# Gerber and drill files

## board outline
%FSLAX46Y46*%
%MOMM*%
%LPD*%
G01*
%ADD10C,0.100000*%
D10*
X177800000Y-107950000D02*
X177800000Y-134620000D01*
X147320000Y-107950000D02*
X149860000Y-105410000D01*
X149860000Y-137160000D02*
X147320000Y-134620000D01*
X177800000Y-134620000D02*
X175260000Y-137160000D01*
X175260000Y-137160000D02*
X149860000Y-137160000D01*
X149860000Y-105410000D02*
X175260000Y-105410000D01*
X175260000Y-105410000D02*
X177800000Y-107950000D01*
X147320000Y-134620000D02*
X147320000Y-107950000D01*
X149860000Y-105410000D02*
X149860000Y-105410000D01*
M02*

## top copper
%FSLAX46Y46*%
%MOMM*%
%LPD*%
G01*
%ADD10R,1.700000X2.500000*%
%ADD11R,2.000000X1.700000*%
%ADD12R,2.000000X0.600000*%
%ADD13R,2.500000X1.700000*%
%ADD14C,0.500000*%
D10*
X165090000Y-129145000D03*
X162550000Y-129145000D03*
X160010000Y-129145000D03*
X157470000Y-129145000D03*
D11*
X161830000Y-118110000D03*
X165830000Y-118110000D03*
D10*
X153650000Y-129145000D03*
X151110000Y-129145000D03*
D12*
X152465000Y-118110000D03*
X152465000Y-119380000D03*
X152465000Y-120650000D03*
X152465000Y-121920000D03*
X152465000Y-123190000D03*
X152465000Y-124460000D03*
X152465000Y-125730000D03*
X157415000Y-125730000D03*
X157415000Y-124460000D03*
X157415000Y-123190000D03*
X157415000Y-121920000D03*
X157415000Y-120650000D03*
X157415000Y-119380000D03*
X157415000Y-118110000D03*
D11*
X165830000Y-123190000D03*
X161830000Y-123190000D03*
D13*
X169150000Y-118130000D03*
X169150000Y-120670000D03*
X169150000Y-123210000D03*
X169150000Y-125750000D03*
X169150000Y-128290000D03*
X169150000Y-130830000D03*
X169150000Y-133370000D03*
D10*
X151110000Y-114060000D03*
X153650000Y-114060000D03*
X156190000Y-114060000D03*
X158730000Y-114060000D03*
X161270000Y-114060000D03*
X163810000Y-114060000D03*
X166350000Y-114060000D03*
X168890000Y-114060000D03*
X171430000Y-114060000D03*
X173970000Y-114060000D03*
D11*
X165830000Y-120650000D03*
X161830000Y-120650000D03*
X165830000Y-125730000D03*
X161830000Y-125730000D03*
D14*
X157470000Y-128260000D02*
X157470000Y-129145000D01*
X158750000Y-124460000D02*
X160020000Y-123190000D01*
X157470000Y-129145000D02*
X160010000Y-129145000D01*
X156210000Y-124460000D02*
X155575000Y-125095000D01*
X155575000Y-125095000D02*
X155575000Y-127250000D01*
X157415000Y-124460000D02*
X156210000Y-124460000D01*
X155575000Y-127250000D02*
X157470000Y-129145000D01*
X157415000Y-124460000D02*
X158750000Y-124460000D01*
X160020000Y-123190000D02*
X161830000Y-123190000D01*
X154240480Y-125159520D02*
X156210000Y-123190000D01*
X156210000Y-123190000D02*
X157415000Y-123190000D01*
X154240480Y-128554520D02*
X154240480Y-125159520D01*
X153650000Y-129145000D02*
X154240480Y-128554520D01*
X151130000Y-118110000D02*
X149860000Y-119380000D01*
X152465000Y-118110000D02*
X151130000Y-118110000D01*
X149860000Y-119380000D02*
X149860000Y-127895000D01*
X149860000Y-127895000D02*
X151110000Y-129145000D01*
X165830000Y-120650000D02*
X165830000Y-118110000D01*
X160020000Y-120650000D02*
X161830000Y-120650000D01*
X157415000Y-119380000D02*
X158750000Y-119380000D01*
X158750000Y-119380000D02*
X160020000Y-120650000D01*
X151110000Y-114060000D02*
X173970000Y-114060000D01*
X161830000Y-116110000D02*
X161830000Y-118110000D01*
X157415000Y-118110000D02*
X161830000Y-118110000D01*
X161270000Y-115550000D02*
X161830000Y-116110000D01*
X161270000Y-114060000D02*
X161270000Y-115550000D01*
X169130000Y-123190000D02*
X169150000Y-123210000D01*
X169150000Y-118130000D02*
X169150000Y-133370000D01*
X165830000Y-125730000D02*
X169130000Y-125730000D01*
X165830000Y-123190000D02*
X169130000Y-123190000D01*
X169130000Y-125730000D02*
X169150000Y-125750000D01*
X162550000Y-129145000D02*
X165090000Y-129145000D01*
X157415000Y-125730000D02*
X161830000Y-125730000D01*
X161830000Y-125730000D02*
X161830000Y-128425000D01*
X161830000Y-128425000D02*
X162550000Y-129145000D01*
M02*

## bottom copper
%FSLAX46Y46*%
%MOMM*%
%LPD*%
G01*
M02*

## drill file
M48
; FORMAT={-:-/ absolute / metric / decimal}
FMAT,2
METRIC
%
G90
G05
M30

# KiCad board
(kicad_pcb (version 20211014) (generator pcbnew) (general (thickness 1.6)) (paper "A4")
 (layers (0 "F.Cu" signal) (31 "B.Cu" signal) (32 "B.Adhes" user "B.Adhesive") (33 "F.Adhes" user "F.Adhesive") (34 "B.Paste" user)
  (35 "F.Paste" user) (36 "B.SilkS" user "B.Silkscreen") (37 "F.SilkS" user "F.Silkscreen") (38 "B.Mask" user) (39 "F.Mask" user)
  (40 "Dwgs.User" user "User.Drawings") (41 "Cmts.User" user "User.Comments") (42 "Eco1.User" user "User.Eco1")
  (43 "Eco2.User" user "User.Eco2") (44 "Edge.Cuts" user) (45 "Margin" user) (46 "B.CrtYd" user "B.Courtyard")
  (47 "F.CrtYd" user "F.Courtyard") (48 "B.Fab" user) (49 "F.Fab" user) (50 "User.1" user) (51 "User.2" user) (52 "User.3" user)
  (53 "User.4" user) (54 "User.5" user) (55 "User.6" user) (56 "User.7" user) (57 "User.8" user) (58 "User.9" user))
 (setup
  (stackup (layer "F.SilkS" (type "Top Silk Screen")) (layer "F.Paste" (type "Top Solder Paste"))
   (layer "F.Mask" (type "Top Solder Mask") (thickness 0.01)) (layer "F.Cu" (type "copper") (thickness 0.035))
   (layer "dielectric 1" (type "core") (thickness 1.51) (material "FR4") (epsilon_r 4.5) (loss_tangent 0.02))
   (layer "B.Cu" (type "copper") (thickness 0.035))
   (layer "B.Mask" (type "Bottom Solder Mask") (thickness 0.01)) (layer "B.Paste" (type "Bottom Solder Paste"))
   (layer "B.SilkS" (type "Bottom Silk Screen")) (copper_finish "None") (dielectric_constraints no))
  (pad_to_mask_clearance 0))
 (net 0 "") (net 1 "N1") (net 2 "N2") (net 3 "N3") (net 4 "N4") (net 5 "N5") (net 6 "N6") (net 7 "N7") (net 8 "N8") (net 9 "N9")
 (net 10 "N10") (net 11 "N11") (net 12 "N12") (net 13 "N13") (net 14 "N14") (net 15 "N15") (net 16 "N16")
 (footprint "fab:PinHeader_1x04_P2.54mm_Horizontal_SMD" (layer "F.Cu") (at 165.09 129.145 -90)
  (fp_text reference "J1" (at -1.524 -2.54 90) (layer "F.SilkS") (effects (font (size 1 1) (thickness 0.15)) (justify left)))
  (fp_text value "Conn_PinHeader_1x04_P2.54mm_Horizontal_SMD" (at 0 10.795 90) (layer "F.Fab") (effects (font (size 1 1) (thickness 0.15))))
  (pad "1" smd rect locked (at 0 0 270) (size 2.5 1.7) (layers "F.Cu" "F.Paste" "F.Mask") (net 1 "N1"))
  (pad "2" smd rect locked (at 0 2.54 270) (size 2.5 1.7) (layers "F.Cu" "F.Paste" "F.Mask") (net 1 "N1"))
  (pad "3" smd rect locked (at 0 5.08 270) (size 2.5 1.7) (layers "F.Cu" "F.Paste" "F.Mask") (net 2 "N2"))
  (pad "4" smd rect locked (at 0 7.62 270) (size 2.5 1.7) (layers "F.Cu" "F.Paste" "F.Mask") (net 2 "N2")))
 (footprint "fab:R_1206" (layer "F.Cu") (at 163.83 118.11)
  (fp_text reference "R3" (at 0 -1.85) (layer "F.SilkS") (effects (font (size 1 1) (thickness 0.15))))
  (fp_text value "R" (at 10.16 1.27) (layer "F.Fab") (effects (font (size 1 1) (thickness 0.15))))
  (pad "1" smd rect locked (at -2 0) (size 2 1.7) (layers "F.Cu" "F.Paste" "F.Mask") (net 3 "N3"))
  (pad "2" smd rect locked (at 2 0) (size 2 1.7) (layers "F.Cu" "F.Paste" "F.Mask") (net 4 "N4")))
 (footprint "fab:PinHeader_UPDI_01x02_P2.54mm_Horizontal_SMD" (layer "F.Cu") (at 153.65 129.145 -90)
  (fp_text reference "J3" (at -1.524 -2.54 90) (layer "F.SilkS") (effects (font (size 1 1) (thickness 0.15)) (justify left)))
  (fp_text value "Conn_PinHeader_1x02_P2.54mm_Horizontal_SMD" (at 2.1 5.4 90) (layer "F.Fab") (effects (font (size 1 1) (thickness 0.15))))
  (pad "1" smd rect locked (at 0 0 270) (size 2.5 1.7) (layers "F.Cu" "F.Paste" "F.Mask") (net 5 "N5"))
  (pad "2" smd rect locked (at 0 2.54 270) (size 2.5 1.7) (layers "F.Cu" "F.Paste" "F.Mask") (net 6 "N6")))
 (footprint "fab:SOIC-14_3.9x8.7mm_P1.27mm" (layer "F.Cu") (at 154.94 121.92)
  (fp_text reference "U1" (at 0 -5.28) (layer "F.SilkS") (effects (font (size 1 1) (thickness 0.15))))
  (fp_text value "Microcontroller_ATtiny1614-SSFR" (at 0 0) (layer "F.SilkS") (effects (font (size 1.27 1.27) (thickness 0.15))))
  (pad "1" smd rect (at -2.475 -3.81) (size 2 0.6) (layers "F.Cu" "F.Paste" "F.Mask") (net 6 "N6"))
  (pad "2" smd rect (at -2.475 -2.54) (size 2 0.6) (layers "F.Cu" "F.Paste" "F.Mask") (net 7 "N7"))
  (pad "3" smd rect (at -2.475 -1.27) (size 2 0.6) (layers "F.Cu" "F.Paste" "F.Mask") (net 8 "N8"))
  (pad "4" smd rect (at -2.475 0) (size 2 0.6) (layers "F.Cu" "F.Paste" "F.Mask") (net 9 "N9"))
  (pad "5" smd rect (at -2.475 1.27) (size 2 0.6) (layers "F.Cu" "F.Paste" "F.Mask") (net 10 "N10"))
  (pad "6" smd rect (at -2.475 2.54) (size 2 0.6) (layers "F.Cu" "F.Paste" "F.Mask") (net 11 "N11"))
  (pad "7" smd rect (at -2.475 3.81) (size 2 0.6) (layers "F.Cu" "F.Paste" "F.Mask") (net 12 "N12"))
  (pad "8" smd rect (at 2.475 3.81) (size 2 0.6) (layers "F.Cu" "F.Paste" "F.Mask") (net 1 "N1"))
  (pad "9" smd rect (at 2.475 2.54) (size 2 0.6) (layers "F.Cu" "F.Paste" "F.Mask") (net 2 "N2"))
  (pad "10" smd rect (at 2.475 1.27) (size 2 0.6) (layers "F.Cu" "F.Paste" "F.Mask") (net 5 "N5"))
  (pad "11" smd rect (at 2.475 0) (size 2 0.6) (layers "F.Cu" "F.Paste" "F.Mask") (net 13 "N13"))
  (pad "12" smd rect (at 2.475 -1.27) (size 2 0.6) (layers "F.Cu" "F.Paste" "F.Mask") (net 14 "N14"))
  (pad "13" smd rect (at 2.475 -2.54) (size 2 0.6) (layers "F.Cu" "F.Paste" "F.Mask") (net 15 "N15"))
  (pad "14" smd rect (at 2.475 -3.81) (size 2 0.6) (layers "F.Cu" "F.Paste" "F.Mask") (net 3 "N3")))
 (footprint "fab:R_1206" (layer "F.Cu") (at 163.83 123.19 180)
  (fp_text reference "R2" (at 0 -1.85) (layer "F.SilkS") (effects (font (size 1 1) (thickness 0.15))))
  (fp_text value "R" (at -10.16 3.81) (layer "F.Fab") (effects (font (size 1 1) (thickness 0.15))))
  (pad "1" smd rect locked (at -2 0 180) (size 2 1.7) (layers "F.Cu" "F.Paste" "F.Mask") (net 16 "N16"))
  (pad "2" smd rect locked (at 2 0 180) (size 2 1.7) (layers "F.Cu" "F.Paste" "F.Mask") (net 2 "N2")))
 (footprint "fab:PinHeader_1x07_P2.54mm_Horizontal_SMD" (layer "F.Cu") (at 169.15 118.13)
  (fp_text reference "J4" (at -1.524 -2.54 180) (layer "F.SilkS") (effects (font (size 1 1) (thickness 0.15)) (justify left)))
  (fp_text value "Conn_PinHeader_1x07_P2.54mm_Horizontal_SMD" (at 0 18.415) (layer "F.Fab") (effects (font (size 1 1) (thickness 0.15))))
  (pad "1" smd rect locked (at 0 0) (size 2.5 1.7) (layers "F.Cu" "F.Paste" "F.Mask") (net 16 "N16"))
  (pad "2" smd rect locked (at 0 2.54) (size 2.5 1.7) (layers "F.Cu" "F.Paste" "F.Mask") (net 16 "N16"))
  (pad "3" smd rect locked (at 0 5.08) (size 2.5 1.7) (layers "F.Cu" "F.Paste" "F.Mask") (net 16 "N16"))
  (pad "4" smd rect locked (at 0 7.62) (size 2.5 1.7) (layers "F.Cu" "F.Paste" "F.Mask") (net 16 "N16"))
  (pad "5" smd rect locked (at 0 10.16) (size 2.5 1.7) (layers "F.Cu" "F.Paste" "F.Mask") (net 16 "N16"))
  (pad "6" smd rect locked (at 0 12.7) (size 2.5 1.7) (layers "F.Cu" "F.Paste" "F.Mask") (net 16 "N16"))
  (pad "7" smd rect locked (at 0 15.24) (size 2.5 1.7) (layers "F.Cu" "F.Paste" "F.Mask") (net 16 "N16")))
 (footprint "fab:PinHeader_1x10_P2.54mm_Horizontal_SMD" (layer "F.Cu") (at 151.11 114.06 90)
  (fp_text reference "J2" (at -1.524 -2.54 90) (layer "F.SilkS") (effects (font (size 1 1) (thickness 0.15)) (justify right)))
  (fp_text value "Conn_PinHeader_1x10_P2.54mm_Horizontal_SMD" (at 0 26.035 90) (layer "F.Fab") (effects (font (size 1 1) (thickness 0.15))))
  (pad "1" smd rect locked (at 0 0 90) (size 2.5 1.7) (layers "F.Cu" "F.Paste" "F.Mask") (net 3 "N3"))
  (pad "2" smd rect locked (at 0 2.54 90) (size 2.5 1.7) (layers "F.Cu" "F.Paste" "F.Mask") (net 3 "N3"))
  (pad "3" smd rect locked (at 0 5.08 90) (size 2.5 1.7) (layers "F.Cu" "F.Paste" "F.Mask") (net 3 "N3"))
  (pad "4" smd rect locked (at 0 7.62 90) (size 2.5 1.7) (layers "F.Cu" "F.Paste" "F.Mask") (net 3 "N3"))
  (pad "5" smd rect locked (at 0 10.16 90) (size 2.5 1.7) (layers "F.Cu" "F.Paste" "F.Mask") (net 3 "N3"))
  (pad "6" smd rect locked (at 0 12.7 90) (size 2.5 1.7) (layers "F.Cu" "F.Paste" "F.Mask") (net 3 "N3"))
  (pad "7" smd rect locked (at 0 15.24 90) (size 2.5 1.7) (layers "F.Cu" "F.Paste" "F.Mask") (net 3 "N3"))
  (pad "8" smd rect locked (at 0 17.78 90) (size 2.5 1.7) (layers "F.Cu" "F.Paste" "F.Mask") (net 3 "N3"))
  (pad "9" smd rect locked (at 0 20.32 90) (size 2.5 1.7) (layers "F.Cu" "F.Paste" "F.Mask") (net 3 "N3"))
  (pad "10" smd rect locked (at 0 22.86 90) (size 2.5 1.7) (layers "F.Cu" "F.Paste" "F.Mask") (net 3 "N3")))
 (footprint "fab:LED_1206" (layer "F.Cu") (at 163.83 120.65 180)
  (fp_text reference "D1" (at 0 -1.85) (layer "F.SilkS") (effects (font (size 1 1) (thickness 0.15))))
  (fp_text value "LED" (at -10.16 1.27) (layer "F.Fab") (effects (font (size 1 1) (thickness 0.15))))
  (pad "1" smd rect locked (at -2 0 180) (size 2 1.7) (layers "F.Cu" "F.Paste" "F.Mask") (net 4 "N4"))
  (pad "2" smd rect locked (at 2 0 180) (size 2 1.7) (layers "F.Cu" "F.Paste" "F.Mask") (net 15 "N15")))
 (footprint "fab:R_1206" (layer "F.Cu") (at 163.83 125.73 180)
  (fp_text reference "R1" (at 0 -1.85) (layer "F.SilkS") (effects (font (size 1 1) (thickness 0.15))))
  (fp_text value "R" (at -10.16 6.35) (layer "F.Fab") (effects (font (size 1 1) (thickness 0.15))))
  (pad "1" smd rect locked (at -2 0 180) (size 2 1.7) (layers "F.Cu" "F.Paste" "F.Mask") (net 16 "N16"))
  (pad "2" smd rect locked (at 2 0 180) (size 2 1.7) (layers "F.Cu" "F.Paste" "F.Mask") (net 1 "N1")))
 (gr_line (start 177.8 107.95) (end 177.8 134.62) (layer "Edge.Cuts") (width 0.1))
 (gr_line (start 147.32 107.95) (end 149.86 105.41) (layer "Edge.Cuts") (width 0.1))
 (gr_line (start 149.86 137.16) (end 147.32 134.62) (layer "Edge.Cuts") (width 0.1))
 (gr_line (start 177.8 134.62) (end 175.26 137.16) (layer "Edge.Cuts") (width 0.1))
 (gr_line (start 175.26 137.16) (end 149.86 137.16) (layer "Edge.Cuts") (width 0.1))
 (gr_line (start 149.86 105.41) (end 175.26 105.41) (layer "Edge.Cuts") (width 0.1))
 (gr_line (start 175.26 105.41) (end 177.8 107.95) (layer "Edge.Cuts") (width 0.1))
 (gr_line (start 147.32 134.62) (end 147.32 107.95) (layer "Edge.Cuts") (width 0.1))
 (gr_line (start 149.86 105.41) (end 149.86 105.41) (layer "Edge.Cuts") (width 0.1))
 (segment (start 157.47 128.26) (end 157.47 129.145) (width 0.5) (layer "F.Cu") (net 2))
 (segment (start 158.75 124.46) (end 160.02 123.19) (width 0.5) (layer "F.Cu") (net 2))
 (segment (start 157.47 129.145) (end 160.01 129.145) (width 0.5) (layer "F.Cu") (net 2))
 (segment (start 156.21 124.46) (end 155.575 125.095) (width 0.5) (layer "F.Cu") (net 2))
 (segment (start 155.575 125.095) (end 155.575 127.25) (width 0.5) (layer "F.Cu") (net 2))
 (segment (start 157.415 124.46) (end 156.21 124.46) (width 0.5) (layer "F.Cu") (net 2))
 (segment (start 155.575 127.25) (end 157.47 129.145) (width 0.5) (layer "F.Cu") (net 2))
 (segment (start 157.415 124.46) (end 158.75 124.46) (width 0.5) (layer "F.Cu") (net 2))
 (segment (start 160.02 123.19) (end 161.83 123.19) (width 0.5) (layer "F.Cu") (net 2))
 (segment (start 154.24048 125.15952) (end 156.21 123.19) (width 0.5) (layer "F.Cu") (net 5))
 (segment (start 156.21 123.19) (end 157.415 123.19) (width 0.5) (layer "F.Cu") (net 5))
 (segment (start 154.24048 128.55452) (end 154.24048 125.15952) (width 0.5) (layer "F.Cu") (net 5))
 (segment (start 153.65 129.145) (end 154.24048 128.55452) (width 0.5) (layer "F.Cu") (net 5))
 (segment (start 151.13 118.11) (end 149.86 119.38) (width 0.5) (layer "F.Cu") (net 6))
 (segment (start 152.465 118.11) (end 151.13 118.11) (width 0.5) (layer "F.Cu") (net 6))
 (segment (start 149.86 119.38) (end 149.86 127.895) (width 0.5) (layer "F.Cu") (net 6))
 (segment (start 149.86 127.895) (end 151.11 129.145) (width 0.5) (layer "F.Cu") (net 6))
 (segment (start 165.83 120.65) (end 165.83 118.11) (width 0.5) (layer "F.Cu") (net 4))
 (segment (start 160.02 120.65) (end 161.83 120.65) (width 0.5) (layer "F.Cu") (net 15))
 (segment (start 157.415 119.38) (end 158.75 119.38) (width 0.5) (layer "F.Cu") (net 15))
 (segment (start 158.75 119.38) (end 160.02 120.65) (width 0.5) (layer "F.Cu") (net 15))
 (segment (start 151.11 114.06) (end 173.97 114.06) (width 0.5) (layer "F.Cu") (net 3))
 (segment (start 161.83 116.11) (end 161.83 118.11) (width 0.5) (layer "F.Cu") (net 3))
 (segment (start 157.415 118.11) (end 161.83 118.11) (width 0.5) (layer "F.Cu") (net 3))
 (segment (start 161.27 115.55) (end 161.83 116.11) (width 0.5) (layer "F.Cu") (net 3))
 (segment (start 161.27 114.06) (end 161.27 115.55) (width 0.5) (layer "F.Cu") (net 3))
 (segment (start 169.13 123.19) (end 169.15 123.21) (width 0.5) (layer "F.Cu") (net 16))
 (segment (start 169.15 118.13) (end 169.15 133.37) (width 0.5) (layer "F.Cu") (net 16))
 (segment (start 165.83 125.73) (end 169.13 125.73) (width 0.5) (layer "F.Cu") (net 16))
 (segment (start 165.83 123.19) (end 169.13 123.19) (width 0.5) (layer "F.Cu") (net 16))
 (segment (start 169.13 125.73) (end 169.15 125.75) (width 0.5) (layer "F.Cu") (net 16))
 (segment (start 162.55 129.145) (end 165.09 129.145) (width 0.5) (layer "F.Cu") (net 1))
 (segment (start 157.415 125.73) (end 161.83 125.73) (width 0.5) (layer "F.Cu") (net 1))
 (segment (start 161.83 125.73) (end 161.83 128.425) (width 0.5) (layer "F.Cu") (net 1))
 (segment (start 161.83 128.425) (end 162.55 129.145) (width 0.5) (layer "F.Cu") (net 1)))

